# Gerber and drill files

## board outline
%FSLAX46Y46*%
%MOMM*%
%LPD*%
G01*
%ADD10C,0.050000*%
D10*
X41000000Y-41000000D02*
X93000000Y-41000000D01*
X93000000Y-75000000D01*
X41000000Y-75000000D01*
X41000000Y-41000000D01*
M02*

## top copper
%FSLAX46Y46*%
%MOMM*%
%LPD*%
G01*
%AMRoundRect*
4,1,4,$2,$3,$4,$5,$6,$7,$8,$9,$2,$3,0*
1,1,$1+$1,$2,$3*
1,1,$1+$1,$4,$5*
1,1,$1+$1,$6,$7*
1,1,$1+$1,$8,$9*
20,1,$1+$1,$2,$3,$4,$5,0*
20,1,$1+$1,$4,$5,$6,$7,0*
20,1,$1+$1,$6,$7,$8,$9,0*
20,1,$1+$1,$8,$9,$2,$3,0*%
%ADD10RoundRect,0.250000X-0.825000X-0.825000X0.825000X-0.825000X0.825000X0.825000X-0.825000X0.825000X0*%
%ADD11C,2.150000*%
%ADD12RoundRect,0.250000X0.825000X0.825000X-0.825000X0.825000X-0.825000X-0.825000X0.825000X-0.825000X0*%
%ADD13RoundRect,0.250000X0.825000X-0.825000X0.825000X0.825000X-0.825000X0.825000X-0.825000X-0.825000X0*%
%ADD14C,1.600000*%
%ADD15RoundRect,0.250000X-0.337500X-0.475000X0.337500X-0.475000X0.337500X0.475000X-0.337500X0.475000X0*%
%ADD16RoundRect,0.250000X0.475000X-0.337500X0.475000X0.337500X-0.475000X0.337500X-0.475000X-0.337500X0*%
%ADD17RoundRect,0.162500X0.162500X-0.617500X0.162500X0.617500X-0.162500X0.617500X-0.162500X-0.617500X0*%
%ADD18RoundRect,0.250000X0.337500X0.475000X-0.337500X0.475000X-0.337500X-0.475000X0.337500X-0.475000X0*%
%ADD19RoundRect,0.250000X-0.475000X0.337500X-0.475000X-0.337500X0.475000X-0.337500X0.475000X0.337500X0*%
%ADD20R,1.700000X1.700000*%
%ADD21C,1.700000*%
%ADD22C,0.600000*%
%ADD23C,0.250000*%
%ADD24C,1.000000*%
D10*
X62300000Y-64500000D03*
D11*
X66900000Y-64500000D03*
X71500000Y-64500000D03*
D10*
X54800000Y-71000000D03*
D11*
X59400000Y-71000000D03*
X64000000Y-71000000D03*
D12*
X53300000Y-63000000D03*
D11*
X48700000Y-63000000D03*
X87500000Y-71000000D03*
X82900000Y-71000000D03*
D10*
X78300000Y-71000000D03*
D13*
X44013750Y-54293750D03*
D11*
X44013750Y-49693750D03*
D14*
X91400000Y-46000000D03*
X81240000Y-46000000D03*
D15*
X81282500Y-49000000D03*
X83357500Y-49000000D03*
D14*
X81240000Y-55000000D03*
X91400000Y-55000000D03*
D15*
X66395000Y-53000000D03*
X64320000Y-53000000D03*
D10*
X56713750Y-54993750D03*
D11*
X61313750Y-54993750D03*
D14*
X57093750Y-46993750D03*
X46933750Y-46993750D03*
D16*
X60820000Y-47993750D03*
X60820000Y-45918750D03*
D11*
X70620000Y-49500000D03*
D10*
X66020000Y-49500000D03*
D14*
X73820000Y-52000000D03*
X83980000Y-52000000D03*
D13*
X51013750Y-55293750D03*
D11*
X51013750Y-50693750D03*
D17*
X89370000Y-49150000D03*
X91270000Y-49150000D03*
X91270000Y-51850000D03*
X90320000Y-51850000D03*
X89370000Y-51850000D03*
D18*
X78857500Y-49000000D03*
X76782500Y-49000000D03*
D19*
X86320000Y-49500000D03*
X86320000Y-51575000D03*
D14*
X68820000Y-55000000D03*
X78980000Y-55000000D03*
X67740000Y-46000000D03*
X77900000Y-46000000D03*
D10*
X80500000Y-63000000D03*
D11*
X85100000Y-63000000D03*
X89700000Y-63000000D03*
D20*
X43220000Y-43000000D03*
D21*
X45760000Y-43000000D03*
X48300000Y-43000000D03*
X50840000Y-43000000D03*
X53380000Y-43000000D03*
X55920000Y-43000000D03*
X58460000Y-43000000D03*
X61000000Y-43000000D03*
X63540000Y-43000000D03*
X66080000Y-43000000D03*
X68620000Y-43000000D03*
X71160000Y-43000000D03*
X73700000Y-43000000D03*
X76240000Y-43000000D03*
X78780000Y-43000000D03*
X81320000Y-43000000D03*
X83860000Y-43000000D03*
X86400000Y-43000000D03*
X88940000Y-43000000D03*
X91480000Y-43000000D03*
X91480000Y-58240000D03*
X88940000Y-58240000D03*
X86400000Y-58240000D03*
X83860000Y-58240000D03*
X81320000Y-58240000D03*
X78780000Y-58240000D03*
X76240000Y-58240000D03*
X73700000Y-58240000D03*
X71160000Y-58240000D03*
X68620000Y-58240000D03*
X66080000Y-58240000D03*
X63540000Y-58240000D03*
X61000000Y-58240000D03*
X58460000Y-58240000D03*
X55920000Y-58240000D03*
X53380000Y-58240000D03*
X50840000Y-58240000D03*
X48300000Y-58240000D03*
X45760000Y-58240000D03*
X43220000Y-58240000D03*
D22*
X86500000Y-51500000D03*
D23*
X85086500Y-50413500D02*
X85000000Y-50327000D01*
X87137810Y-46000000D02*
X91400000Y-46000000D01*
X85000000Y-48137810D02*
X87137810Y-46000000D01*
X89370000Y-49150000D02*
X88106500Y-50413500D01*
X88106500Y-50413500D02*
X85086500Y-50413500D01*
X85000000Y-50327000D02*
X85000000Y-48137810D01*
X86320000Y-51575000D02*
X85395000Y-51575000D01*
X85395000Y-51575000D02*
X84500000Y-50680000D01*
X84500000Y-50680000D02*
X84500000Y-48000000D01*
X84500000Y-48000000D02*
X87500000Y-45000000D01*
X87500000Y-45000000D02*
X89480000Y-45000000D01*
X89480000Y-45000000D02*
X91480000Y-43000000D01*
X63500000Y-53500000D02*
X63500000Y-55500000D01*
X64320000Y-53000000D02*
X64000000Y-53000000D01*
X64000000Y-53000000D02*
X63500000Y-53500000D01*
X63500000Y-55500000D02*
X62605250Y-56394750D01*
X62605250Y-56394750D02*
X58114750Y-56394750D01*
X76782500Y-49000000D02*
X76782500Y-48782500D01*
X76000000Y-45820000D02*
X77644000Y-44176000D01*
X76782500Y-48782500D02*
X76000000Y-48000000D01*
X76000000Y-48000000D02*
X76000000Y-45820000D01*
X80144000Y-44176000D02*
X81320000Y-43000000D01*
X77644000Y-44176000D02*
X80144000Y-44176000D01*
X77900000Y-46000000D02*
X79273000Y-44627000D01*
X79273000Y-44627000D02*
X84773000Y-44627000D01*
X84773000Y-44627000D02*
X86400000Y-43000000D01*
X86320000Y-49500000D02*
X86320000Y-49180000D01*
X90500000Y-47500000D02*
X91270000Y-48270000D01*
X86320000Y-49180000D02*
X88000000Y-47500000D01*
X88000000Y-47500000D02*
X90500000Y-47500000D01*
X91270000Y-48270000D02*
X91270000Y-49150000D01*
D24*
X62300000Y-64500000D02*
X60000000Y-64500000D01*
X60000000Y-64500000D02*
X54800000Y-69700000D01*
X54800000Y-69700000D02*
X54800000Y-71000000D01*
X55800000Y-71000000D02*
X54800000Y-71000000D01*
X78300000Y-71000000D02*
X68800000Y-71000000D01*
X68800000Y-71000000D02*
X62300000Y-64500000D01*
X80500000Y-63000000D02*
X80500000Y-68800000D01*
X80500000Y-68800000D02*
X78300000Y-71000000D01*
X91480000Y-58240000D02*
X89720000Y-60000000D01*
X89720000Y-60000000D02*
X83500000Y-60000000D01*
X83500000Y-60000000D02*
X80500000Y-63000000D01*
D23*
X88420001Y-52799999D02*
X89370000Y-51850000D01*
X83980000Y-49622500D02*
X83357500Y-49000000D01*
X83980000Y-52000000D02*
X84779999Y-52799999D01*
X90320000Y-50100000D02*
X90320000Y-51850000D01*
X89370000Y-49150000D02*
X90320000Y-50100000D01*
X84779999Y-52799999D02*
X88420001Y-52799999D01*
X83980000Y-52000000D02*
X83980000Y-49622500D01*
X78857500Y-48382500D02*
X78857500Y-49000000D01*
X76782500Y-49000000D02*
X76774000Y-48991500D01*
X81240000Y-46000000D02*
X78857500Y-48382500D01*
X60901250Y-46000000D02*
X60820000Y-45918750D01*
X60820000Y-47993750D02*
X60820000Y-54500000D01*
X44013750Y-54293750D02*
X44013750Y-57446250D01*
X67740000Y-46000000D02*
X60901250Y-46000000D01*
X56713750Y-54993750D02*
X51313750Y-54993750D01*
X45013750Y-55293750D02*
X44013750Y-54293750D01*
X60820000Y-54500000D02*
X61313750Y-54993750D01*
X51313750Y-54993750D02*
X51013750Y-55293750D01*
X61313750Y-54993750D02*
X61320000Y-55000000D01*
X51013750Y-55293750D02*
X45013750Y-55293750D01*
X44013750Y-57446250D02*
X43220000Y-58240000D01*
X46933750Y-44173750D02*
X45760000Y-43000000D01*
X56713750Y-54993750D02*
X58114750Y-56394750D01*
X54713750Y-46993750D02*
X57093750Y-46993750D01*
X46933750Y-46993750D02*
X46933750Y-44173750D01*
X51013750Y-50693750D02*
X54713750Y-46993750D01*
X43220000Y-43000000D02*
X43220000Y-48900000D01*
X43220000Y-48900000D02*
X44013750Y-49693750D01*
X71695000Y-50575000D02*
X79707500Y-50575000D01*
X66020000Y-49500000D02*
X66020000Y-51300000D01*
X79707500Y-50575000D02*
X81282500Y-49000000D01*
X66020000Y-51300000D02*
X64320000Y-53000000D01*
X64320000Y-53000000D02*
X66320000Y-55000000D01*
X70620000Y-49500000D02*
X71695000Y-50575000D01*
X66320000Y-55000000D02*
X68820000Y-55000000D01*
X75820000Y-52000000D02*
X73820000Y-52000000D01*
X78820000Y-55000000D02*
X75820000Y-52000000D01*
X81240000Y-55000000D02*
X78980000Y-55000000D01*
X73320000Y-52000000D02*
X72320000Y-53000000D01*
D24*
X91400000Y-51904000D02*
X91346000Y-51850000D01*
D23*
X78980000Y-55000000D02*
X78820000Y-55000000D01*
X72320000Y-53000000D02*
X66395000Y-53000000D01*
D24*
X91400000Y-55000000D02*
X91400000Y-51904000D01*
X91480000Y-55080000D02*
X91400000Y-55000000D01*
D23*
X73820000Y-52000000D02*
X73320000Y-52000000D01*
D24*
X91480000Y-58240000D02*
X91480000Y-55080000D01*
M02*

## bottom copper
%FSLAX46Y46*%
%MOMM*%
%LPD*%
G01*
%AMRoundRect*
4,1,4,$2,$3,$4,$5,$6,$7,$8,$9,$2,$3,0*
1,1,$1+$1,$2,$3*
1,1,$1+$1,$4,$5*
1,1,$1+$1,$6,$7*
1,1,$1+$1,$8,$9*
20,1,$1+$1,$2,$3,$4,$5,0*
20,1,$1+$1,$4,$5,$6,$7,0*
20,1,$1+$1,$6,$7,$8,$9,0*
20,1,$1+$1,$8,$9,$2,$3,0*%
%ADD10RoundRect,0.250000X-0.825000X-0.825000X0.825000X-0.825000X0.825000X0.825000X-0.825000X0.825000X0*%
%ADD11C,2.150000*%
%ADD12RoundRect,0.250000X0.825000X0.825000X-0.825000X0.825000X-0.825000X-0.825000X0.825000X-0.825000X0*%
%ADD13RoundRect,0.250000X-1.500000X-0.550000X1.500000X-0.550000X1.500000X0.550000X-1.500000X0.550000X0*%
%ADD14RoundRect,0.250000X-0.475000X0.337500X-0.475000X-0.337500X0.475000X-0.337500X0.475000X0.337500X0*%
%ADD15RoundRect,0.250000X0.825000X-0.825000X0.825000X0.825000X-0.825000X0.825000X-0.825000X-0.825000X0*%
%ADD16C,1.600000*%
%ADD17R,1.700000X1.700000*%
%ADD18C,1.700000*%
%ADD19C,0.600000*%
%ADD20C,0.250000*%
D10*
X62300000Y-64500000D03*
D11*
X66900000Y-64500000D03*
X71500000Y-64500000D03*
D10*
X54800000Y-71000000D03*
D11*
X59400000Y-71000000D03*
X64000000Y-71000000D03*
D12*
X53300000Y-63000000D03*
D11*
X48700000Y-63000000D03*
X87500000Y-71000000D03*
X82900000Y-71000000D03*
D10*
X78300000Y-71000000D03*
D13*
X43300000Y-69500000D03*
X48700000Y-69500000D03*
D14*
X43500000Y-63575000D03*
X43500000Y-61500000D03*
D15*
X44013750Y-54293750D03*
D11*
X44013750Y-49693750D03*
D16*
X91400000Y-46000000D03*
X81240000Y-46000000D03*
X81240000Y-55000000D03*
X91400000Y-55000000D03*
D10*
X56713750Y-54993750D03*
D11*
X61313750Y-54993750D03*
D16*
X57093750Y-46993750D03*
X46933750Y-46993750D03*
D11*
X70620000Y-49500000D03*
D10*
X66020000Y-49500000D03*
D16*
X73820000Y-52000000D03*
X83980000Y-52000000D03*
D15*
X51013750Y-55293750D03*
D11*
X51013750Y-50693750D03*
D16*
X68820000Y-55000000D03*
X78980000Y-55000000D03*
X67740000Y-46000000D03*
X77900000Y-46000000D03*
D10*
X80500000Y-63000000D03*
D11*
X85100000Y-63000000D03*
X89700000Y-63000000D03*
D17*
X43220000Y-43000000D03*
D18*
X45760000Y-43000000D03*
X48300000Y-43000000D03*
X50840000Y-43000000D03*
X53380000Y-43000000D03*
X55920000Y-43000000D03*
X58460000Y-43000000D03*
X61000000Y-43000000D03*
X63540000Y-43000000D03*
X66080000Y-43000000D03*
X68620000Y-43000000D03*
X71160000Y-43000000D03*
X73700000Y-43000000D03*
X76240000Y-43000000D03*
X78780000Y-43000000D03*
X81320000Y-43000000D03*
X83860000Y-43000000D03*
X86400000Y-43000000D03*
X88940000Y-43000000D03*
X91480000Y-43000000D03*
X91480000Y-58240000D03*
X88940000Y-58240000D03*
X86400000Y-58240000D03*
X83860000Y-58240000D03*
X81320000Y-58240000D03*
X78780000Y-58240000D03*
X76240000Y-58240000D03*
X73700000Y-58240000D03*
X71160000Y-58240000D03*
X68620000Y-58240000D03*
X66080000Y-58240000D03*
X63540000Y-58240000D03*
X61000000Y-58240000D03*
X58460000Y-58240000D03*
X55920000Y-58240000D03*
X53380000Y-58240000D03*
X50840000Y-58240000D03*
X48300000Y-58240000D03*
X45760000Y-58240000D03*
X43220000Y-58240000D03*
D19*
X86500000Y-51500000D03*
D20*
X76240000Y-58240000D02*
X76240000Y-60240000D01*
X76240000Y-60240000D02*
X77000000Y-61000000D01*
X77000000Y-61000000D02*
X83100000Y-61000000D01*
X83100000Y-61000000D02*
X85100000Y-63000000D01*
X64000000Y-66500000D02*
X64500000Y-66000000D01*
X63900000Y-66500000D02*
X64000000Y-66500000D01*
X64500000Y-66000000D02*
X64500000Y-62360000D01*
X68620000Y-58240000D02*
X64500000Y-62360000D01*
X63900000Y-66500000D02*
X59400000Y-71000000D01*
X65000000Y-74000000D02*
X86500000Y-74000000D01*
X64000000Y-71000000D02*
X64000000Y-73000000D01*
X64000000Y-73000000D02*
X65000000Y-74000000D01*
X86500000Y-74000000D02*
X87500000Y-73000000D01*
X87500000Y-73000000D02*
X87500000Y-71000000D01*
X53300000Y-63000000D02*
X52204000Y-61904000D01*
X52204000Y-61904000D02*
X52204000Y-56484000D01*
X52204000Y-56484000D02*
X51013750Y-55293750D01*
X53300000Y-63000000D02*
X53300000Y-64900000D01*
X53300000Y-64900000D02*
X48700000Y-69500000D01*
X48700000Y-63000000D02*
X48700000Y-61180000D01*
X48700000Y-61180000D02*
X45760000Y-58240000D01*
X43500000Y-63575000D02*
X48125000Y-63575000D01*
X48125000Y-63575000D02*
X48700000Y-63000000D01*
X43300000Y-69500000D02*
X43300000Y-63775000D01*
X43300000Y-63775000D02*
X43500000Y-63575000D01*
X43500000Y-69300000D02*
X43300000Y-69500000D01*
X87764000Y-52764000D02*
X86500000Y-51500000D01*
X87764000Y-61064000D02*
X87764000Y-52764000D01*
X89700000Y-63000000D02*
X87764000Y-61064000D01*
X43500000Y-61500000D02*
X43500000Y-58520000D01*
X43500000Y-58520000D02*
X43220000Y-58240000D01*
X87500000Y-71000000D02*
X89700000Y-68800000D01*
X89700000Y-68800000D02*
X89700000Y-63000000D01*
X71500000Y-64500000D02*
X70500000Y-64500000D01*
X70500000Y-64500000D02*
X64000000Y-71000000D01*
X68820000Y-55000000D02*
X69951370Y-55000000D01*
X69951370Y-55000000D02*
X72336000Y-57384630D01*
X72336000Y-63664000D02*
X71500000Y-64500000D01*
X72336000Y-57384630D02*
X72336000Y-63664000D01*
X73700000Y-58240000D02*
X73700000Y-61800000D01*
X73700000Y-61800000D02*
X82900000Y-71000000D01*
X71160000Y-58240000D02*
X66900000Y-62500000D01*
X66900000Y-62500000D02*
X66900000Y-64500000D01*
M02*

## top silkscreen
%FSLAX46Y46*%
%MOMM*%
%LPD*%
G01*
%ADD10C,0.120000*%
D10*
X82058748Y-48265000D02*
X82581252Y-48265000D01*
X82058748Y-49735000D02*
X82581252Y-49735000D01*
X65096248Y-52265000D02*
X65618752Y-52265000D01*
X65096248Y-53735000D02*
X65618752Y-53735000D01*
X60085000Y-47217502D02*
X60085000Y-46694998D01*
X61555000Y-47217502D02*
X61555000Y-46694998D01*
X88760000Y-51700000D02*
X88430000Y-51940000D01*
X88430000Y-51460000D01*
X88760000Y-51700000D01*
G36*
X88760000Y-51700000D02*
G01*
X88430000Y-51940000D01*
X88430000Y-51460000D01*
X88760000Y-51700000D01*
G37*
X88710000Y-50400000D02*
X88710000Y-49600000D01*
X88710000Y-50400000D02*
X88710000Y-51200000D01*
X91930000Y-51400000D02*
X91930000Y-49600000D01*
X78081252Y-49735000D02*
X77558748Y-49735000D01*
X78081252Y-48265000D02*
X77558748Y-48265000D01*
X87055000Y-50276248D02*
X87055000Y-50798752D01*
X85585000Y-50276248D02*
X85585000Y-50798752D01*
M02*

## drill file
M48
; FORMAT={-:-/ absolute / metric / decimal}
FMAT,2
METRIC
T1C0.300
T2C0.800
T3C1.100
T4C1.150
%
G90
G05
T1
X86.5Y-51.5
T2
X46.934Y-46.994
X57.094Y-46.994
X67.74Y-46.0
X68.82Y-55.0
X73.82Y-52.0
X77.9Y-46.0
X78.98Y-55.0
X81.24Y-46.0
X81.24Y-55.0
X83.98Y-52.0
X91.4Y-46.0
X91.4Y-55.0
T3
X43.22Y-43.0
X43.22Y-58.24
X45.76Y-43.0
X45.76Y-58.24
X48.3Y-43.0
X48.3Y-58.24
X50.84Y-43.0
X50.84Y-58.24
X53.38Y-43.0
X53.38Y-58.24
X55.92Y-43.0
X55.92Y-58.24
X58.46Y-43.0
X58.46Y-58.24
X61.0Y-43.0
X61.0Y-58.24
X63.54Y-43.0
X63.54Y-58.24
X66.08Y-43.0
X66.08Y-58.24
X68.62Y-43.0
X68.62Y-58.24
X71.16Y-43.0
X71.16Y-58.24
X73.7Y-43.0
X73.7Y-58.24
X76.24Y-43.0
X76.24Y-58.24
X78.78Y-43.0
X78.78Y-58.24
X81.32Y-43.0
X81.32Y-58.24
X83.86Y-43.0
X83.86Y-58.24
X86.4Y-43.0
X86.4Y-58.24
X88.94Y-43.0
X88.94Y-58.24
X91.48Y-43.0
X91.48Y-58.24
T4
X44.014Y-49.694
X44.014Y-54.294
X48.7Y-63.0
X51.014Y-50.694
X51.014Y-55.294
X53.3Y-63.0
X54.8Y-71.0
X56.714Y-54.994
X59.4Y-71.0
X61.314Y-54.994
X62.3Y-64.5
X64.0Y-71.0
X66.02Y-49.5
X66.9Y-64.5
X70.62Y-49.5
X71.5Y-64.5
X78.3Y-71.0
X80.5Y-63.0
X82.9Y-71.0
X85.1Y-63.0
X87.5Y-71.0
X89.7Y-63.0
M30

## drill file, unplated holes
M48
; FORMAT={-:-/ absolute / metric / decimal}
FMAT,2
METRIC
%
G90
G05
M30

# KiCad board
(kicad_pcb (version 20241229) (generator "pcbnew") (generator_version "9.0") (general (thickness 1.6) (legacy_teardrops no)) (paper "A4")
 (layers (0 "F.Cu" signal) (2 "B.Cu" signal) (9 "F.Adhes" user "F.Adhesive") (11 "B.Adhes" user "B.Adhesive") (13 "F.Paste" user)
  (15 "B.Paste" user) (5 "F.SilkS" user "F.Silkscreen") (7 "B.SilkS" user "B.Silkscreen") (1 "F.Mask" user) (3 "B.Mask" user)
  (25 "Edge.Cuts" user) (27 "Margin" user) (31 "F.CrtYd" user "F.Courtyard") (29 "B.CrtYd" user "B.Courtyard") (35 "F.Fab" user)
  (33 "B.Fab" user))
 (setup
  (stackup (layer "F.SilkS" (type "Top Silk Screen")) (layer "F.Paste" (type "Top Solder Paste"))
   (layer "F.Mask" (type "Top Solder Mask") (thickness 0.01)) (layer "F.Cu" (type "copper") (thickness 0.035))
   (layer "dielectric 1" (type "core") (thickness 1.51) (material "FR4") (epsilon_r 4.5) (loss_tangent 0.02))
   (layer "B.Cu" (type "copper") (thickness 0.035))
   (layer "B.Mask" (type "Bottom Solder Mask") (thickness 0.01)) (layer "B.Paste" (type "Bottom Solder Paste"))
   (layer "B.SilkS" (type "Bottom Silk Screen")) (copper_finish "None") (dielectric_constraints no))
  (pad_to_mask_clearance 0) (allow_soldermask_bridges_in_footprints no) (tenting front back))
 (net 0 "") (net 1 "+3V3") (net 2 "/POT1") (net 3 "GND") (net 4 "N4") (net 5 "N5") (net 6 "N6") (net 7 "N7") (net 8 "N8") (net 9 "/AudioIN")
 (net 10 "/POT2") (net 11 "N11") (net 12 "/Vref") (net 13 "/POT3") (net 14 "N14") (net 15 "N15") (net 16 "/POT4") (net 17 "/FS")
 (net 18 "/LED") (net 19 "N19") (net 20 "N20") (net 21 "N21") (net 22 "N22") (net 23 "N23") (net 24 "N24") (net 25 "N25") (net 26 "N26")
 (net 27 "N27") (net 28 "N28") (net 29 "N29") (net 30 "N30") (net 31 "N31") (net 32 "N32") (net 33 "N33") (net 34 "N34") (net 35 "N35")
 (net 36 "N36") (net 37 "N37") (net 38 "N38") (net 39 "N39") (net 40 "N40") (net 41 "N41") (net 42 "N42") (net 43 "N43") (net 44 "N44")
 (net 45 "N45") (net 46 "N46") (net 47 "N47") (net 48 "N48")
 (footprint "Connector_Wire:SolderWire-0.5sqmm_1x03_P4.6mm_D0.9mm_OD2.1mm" (layer "F.Cu") (at 54.8 71)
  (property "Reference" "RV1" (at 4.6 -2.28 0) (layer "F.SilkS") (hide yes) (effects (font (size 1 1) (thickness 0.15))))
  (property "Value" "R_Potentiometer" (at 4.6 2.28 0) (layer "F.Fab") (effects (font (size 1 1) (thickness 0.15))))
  (pad "1" thru_hole roundrect (at 0 0) (size 2.15 2.15) (drill 1.15) (layers "*.Cu" "*.Mask") (remove_unused_layers no)
   (roundrect_rratio 0.116279) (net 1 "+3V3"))
  (pad "2" thru_hole circle (at 4.6 0) (size 2.15 2.15) (drill 1.15) (layers "*.Cu" "*.Mask") (remove_unused_layers no) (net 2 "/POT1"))
  (pad "3" thru_hole circle (at 9.2 0) (size 2.15 2.15) (drill 1.15) (layers "*.Cu" "*.Mask") (remove_unused_layers no) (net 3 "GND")))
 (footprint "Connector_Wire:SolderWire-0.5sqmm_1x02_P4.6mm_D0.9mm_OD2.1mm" (layer "F.Cu") (at 53.3 63 180)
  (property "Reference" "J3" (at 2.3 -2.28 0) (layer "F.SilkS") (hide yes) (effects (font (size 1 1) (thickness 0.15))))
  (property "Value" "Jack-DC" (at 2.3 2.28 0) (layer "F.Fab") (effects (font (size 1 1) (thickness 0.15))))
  (pad "1" thru_hole roundrect (at 0 0 180) (size 2.15 2.15) (drill 1.15) (layers "*.Cu" "*.Mask") (remove_unused_layers no)
   (roundrect_rratio 0.116279) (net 3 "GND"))
  (pad "2" thru_hole circle (at 4.6 0 180) (size 2.15 2.15) (drill 1.15) (layers "*.Cu" "*.Mask") (remove_unused_layers no) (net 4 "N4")))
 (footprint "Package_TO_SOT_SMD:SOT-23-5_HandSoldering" (layer "F.Cu") (at 90.32 50.5 90)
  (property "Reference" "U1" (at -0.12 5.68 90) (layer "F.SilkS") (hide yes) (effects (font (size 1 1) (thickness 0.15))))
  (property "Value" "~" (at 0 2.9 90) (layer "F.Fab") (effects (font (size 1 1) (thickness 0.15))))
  (fp_line (start 0.1 -1.61) (end 0.9 -1.61) (stroke (width 0.12) (type solid)) (layer "F.SilkS"))
  (fp_line (start 0.1 -1.61) (end -0.7 -1.61) (stroke (width 0.12) (type solid)) (layer "F.SilkS"))
  (fp_line (start -0.9 1.61) (end 0.9 1.61) (stroke (width 0.12) (type solid)) (layer "F.SilkS"))
  (fp_poly
   (pts (xy -1.2 -1.56) (xy -1.44 -1.89) (xy -0.96 -1.89) (xy -1.2 -1.56)) (stroke (width 0.12) (type solid)) (fill yes) (layer "F.SilkS"))
  (pad "1" smd roundrect (at -1.35 -0.95 90) (size 1.56 0.65) (layers "F.Cu" "F.Mask" "F.Paste") (roundrect_rratio 0.25) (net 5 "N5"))
  (pad "2" smd roundrect (at -1.35 0 90) (size 1.56 0.65) (layers "F.Cu" "F.Mask" "F.Paste") (roundrect_rratio 0.25) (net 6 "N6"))
  (pad "3" smd roundrect (at -1.35 0.95 90) (size 1.56 0.65) (layers "F.Cu" "F.Mask" "F.Paste") (roundrect_rratio 0.25) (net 1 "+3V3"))
  (pad "4" smd roundrect (at 1.35 0.95 90) (size 1.56 0.65) (layers "F.Cu" "F.Mask" "F.Paste") (roundrect_rratio 0.25) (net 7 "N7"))
  (pad "5" smd roundrect (at 1.35 -0.95 90) (size 1.56 0.65) (layers "F.Cu" "F.Mask" "F.Paste") (roundrect_rratio 0.25) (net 6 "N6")))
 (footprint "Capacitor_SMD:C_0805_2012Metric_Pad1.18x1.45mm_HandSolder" (layer "F.Cu") (at 77.82 49 180)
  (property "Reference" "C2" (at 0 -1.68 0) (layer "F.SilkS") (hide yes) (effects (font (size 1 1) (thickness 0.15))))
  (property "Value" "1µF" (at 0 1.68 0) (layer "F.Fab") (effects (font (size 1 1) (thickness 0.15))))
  (fp_line (start -0.261252 0.735) (end 0.261252 0.735) (stroke (width 0.12) (type solid)) (layer "F.SilkS"))
  (fp_line (start -0.261252 -0.735) (end 0.261252 -0.735) (stroke (width 0.12) (type solid)) (layer "F.SilkS"))
  (pad "1" smd roundrect (at -1.0375 0 180) (size 1.175 1.45) (layers "F.Cu" "F.Mask" "F.Paste") (roundrect_rratio 0.212766) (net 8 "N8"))
  (pad "2" smd roundrect (at 1.0375 0 180) (size 1.175 1.45) (layers "F.Cu" "F.Mask" "F.Paste") (roundrect_rratio 0.212766)
   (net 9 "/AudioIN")))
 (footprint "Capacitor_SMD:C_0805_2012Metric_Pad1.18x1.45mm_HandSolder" (layer "F.Cu") (at 86.32 50.5375 -90)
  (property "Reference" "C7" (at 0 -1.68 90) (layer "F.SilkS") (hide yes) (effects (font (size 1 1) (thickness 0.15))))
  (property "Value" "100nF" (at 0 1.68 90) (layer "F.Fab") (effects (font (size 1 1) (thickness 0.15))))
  (fp_line (start -0.261252 0.735) (end 0.261252 0.735) (stroke (width 0.12) (type solid)) (layer "F.SilkS"))
  (fp_line (start -0.261252 -0.735) (end 0.261252 -0.735) (stroke (width 0.12) (type solid)) (layer "F.SilkS"))
  (pad "1" smd roundrect (at -1.0375 0 270) (size 1.175 1.45) (layers "F.Cu" "F.Mask" "F.Paste") (roundrect_rratio 0.212766) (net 7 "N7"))
  (pad "2" smd roundrect (at 1.0375 0 270) (size 1.175 1.45) (layers "F.Cu" "F.Mask" "F.Paste") (roundrect_rratio 0.212766) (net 3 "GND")))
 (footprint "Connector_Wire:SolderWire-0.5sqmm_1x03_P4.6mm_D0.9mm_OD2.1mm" (layer "F.Cu") (at 62.3 64.5)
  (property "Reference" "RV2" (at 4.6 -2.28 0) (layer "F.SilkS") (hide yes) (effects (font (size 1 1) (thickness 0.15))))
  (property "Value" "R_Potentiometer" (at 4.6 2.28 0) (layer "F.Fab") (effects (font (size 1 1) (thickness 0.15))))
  (pad "1" thru_hole roundrect (at 0 0) (size 2.15 2.15) (drill 1.15) (layers "*.Cu" "*.Mask") (remove_unused_layers no)
   (roundrect_rratio 0.116279) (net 1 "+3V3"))
  (pad "2" thru_hole circle (at 4.6 0) (size 2.15 2.15) (drill 1.15) (layers "*.Cu" "*.Mask") (remove_unused_layers no) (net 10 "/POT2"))
  (pad "3" thru_hole circle (at 9.2 0) (size 2.15 2.15) (drill 1.15) (layers "*.Cu" "*.Mask") (remove_unused_layers no) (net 3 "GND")))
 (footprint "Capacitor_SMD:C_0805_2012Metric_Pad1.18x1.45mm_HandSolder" (layer "F.Cu") (at 82.32 49)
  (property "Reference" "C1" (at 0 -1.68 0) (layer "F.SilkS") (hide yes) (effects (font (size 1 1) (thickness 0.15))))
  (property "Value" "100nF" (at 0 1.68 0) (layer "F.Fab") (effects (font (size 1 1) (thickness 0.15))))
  (fp_line (start -0.261252 -0.735) (end 0.261252 -0.735) (stroke (width 0.12) (type solid)) (layer "F.SilkS"))
  (fp_line (start -0.261252 0.735) (end 0.261252 0.735) (stroke (width 0.12) (type solid)) (layer "F.SilkS"))
  (pad "1" smd roundrect (at -1.0375 0) (size 1.175 1.45) (layers "F.Cu" "F.Mask" "F.Paste") (roundrect_rratio 0.212766) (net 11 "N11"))
  (pad "2" smd roundrect (at 1.0375 0) (size 1.175 1.45) (layers "F.Cu" "F.Mask" "F.Paste") (roundrect_rratio 0.212766) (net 5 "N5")))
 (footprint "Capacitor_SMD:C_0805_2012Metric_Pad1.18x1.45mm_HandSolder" (layer "F.Cu") (at 65.3575 53)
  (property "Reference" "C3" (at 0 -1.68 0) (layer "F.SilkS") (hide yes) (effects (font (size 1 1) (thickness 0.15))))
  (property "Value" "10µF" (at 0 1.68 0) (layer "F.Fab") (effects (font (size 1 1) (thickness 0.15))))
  (fp_line (start -0.261252 -0.735) (end 0.261252 -0.735) (stroke (width 0.12) (type solid)) (layer "F.SilkS"))
  (fp_line (start -0.261252 0.735) (end 0.261252 0.735) (stroke (width 0.12) (type solid)) (layer "F.SilkS"))
  (pad "1" smd roundrect (at -1.0375 0) (size 1.175 1.45) (layers "F.Cu" "F.Mask" "F.Paste") (roundrect_rratio 0.212766) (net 3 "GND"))
  (pad "2" smd roundrect (at 1.0375 0) (size 1.175 1.45) (layers "F.Cu" "F.Mask" "F.Paste") (roundrect_rratio 0.212766) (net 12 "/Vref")))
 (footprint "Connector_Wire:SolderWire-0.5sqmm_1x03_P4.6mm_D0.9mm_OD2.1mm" (layer "F.Cu") (at 78.3 71)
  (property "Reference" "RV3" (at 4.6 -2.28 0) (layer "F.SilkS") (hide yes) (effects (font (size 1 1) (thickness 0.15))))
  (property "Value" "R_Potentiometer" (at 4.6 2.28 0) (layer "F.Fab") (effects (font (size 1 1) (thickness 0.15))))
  (pad "1" thru_hole roundrect (at 0 0) (size 2.15 2.15) (drill 1.15) (layers "*.Cu" "*.Mask") (remove_unused_layers no)
   (roundrect_rratio 0.116279) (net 1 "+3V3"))
  (pad "2" thru_hole circle (at 4.6 0) (size 2.15 2.15) (drill 1.15) (layers "*.Cu" "*.Mask") (remove_unused_layers no) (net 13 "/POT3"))
  (pad "3" thru_hole circle (at 9.2 0) (size 2.15 2.15) (drill 1.15) (layers "*.Cu" "*.Mask") (remove_unused_layers no) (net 3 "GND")))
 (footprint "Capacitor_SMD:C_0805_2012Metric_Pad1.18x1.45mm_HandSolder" (layer "F.Cu") (at 60.82 46.95625 90)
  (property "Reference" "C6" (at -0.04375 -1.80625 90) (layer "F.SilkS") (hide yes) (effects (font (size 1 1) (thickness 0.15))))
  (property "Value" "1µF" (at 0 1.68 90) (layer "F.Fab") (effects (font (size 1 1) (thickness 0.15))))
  (fp_line (start -0.261252 -0.735) (end 0.261252 -0.735) (stroke (width 0.12) (type solid)) (layer "F.SilkS"))
  (fp_line (start -0.261252 0.735) (end 0.261252 0.735) (stroke (width 0.12) (type solid)) (layer "F.SilkS"))
  (pad "1" smd roundrect (at -1.0375 0 90) (size 1.175 1.45) (layers "F.Cu" "F.Mask" "F.Paste") (roundrect_rratio 0.212766) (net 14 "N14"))
  (pad "2" smd roundrect (at 1.0375 0 90) (size 1.175 1.45) (layers "F.Cu" "F.Mask" "F.Paste") (roundrect_rratio 0.212766) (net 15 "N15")))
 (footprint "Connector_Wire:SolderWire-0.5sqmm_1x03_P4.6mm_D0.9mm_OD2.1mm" (layer "F.Cu") (at 80.5 63)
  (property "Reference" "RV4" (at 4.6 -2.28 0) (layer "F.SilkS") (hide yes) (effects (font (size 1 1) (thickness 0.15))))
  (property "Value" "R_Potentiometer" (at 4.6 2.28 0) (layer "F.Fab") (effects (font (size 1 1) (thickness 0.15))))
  (pad "1" thru_hole roundrect (at 0 0) (size 2.15 2.15) (drill 1.15) (layers "*.Cu" "*.Mask") (remove_unused_layers no)
   (roundrect_rratio 0.116279) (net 1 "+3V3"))
  (pad "2" thru_hole circle (at 4.6 0) (size 2.15 2.15) (drill 1.15) (layers "*.Cu" "*.Mask") (remove_unused_layers no) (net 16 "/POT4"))
  (pad "3" thru_hole circle (at 9.2 0) (size 2.15 2.15) (drill 1.15) (layers "*.Cu" "*.Mask") (remove_unused_layers no) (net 3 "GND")))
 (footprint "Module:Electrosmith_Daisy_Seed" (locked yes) (layer "B.Cu") (at 43.22 43 -90)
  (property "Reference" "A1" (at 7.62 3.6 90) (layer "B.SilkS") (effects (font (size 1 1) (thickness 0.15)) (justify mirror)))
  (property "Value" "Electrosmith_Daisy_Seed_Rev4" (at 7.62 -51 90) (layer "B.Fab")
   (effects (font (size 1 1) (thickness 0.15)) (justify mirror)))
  (pad "1" thru_hole rect (at 0 0 270) (size 1.7 1.7) (drill 1.1) (layers "*.Cu" "*.Mask") (remove_unused_layers no) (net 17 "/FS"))
  (pad "2" thru_hole circle (at 0 -2.54 270) (size 1.7 1.7) (drill 1.1) (layers "*.Cu" "*.Mask") (remove_unused_layers no) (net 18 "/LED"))
  (pad "3" thru_hole circle (at 0 -5.08 270) (size 1.7 1.7) (drill 1.1) (layers "*.Cu" "*.Mask") (remove_unused_layers no) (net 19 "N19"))
  (pad "4" thru_hole circle (at 0 -7.62 270) (size 1.7 1.7) (drill 1.1) (layers "*.Cu" "*.Mask") (remove_unused_layers no) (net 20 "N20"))
  (pad "5" thru_hole circle (at 0 -10.16 270) (size 1.7 1.7) (drill 1.1) (layers "*.Cu" "*.Mask") (remove_unused_layers no) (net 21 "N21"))
  (pad "6" thru_hole circle (at 0 -12.7 270) (size 1.7 1.7) (drill 1.1) (layers "*.Cu" "*.Mask") (remove_unused_layers no) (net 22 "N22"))
  (pad "7" thru_hole circle (at 0 -15.24 270) (size 1.7 1.7) (drill 1.1) (layers "*.Cu" "*.Mask") (remove_unused_layers no) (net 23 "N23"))
  (pad "8" thru_hole circle (at 0 -17.78 270) (size 1.7 1.7) (drill 1.1) (layers "*.Cu" "*.Mask") (remove_unused_layers no) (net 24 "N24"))
  (pad "9" thru_hole circle (at 0 -20.32 270) (size 1.7 1.7) (drill 1.1) (layers "*.Cu" "*.Mask") (remove_unused_layers no) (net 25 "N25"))
  (pad "10" thru_hole circle (at 0 -22.86 270) (size 1.7 1.7) (drill 1.1) (layers "*.Cu" "*.Mask") (remove_unused_layers no) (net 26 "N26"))
  (pad "11" thru_hole circle (at 0 -25.4 270) (size 1.7 1.7) (drill 1.1) (layers "*.Cu" "*.Mask") (remove_unused_layers no) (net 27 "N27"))
  (pad "12" thru_hole circle (at 0 -27.94 270) (size 1.7 1.7) (drill 1.1) (layers "*.Cu" "*.Mask") (remove_unused_layers no) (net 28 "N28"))
  (pad "13" thru_hole circle (at 0 -30.48 270) (size 1.7 1.7) (drill 1.1) (layers "*.Cu" "*.Mask") (remove_unused_layers no) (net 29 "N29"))
  (pad "14" thru_hole circle (at 0 -33.02 270) (size 1.7 1.7) (drill 1.1) (layers "*.Cu" "*.Mask") (remove_unused_layers no) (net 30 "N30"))
  (pad "15" thru_hole circle (at 0 -35.56 270) (size 1.7 1.7) (drill 1.1) (layers "*.Cu" "*.Mask") (remove_unused_layers no) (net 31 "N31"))
  (pad "16" thru_hole circle (at 0 -38.1 270) (size 1.7 1.7) (drill 1.1) (layers "*.Cu" "*.Mask") (remove_unused_layers no)
   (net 9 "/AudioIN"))
  (pad "17" thru_hole circle (at 0 -40.64 270) (size 1.7 1.7) (drill 1.1) (layers "*.Cu" "*.Mask") (remove_unused_layers no) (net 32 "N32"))
  (pad "18" thru_hole circle (at 0 -43.18 270) (size 1.7 1.7) (drill 1.1) (layers "*.Cu" "*.Mask") (remove_unused_layers no) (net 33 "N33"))
  (pad "19" thru_hole circle (at 0 -45.72 270) (size 1.7 1.7) (drill 1.1) (layers "*.Cu" "*.Mask") (remove_unused_layers no) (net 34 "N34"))
  (pad "20" thru_hole circle (at 0 -48.26 270) (size 1.7 1.7) (drill 1.1) (layers "*.Cu" "*.Mask") (remove_unused_layers no) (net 3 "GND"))
  (pad "21" thru_hole circle (at 15.24 -48.26 270) (size 1.7 1.7) (drill 1.1) (layers "*.Cu" "*.Mask") (remove_unused_layers no)
   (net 1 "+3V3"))
  (pad "22" thru_hole circle (at 15.24 -45.72 270) (size 1.7 1.7) (drill 1.1) (layers "*.Cu" "*.Mask") (remove_unused_layers no)
   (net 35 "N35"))
  (pad "23" thru_hole circle (at 15.24 -43.18 270) (size 1.7 1.7) (drill 1.1) (layers "*.Cu" "*.Mask") (remove_unused_layers no)
   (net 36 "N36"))
  (pad "24" thru_hole circle (at 15.24 -40.64 270) (size 1.7 1.7) (drill 1.1) (layers "*.Cu" "*.Mask") (remove_unused_layers no)
   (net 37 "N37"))
  (pad "25" thru_hole circle (at 15.24 -38.1 270) (size 1.7 1.7) (drill 1.1) (layers "*.Cu" "*.Mask") (remove_unused_layers no)
   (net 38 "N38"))
  (pad "26" thru_hole circle (at 15.24 -35.56 270) (size 1.7 1.7) (drill 1.1) (layers "*.Cu" "*.Mask") (remove_unused_layers no)
   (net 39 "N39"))
  (pad "27" thru_hole circle (at 15.24 -33.02 270) (size 1.7 1.7) (drill 1.1) (layers "*.Cu" "*.Mask") (remove_unused_layers no)
   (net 16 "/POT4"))
  (pad "28" thru_hole circle (at 15.24 -30.48 270) (size 1.7 1.7) (drill 1.1) (layers "*.Cu" "*.Mask") (remove_unused_layers no)
   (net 13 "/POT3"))
  (pad "29" thru_hole circle (at 15.24 -27.94 270) (size 1.7 1.7) (drill 1.1) (layers "*.Cu" "*.Mask") (remove_unused_layers no)
   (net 10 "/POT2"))
  (pad "30" thru_hole circle (at 15.24 -25.4 270) (size 1.7 1.7) (drill 1.1) (layers "*.Cu" "*.Mask") (remove_unused_layers no)
   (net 2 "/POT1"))
  (pad "31" thru_hole circle (at 15.24 -22.86 270) (size 1.7 1.7) (drill 1.1) (layers "*.Cu" "*.Mask") (remove_unused_layers no)
   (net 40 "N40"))
  (pad "32" thru_hole circle (at 15.24 -20.32 270) (size 1.7 1.7) (drill 1.1) (layers "*.Cu" "*.Mask") (remove_unused_layers no)
   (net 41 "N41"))
  (pad "33" thru_hole circle (at 15.24 -17.78 270) (size 1.7 1.7) (drill 1.1) (layers "*.Cu" "*.Mask") (remove_unused_layers no)
   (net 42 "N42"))
  (pad "34" thru_hole circle (at 15.24 -15.24 270) (size 1.7 1.7) (drill 1.1) (layers "*.Cu" "*.Mask") (remove_unused_layers no)
   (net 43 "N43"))
  (pad "35" thru_hole circle (at 15.24 -12.7 270) (size 1.7 1.7) (drill 1.1) (layers "*.Cu" "*.Mask") (remove_unused_layers no)
   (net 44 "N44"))
  (pad "36" thru_hole circle (at 15.24 -10.16 270) (size 1.7 1.7) (drill 1.1) (layers "*.Cu" "*.Mask") (remove_unused_layers no)
   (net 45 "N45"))
  (pad "37" thru_hole circle (at 15.24 -7.62 270) (size 1.7 1.7) (drill 1.1) (layers "*.Cu" "*.Mask") (remove_unused_layers no)
   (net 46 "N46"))
  (pad "38" thru_hole circle (at 15.24 -5.08 270) (size 1.7 1.7) (drill 1.1) (layers "*.Cu" "*.Mask") (remove_unused_layers no)
   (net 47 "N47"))
  (pad "39" thru_hole circle (at 15.24 -2.54 270) (size 1.7 1.7) (drill 1.1) (layers "*.Cu" "*.Mask") (remove_unused_layers no) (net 4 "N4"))
  (pad "40" thru_hole circle (at 15.24 0 270) (size 1.7 1.7) (drill 1.1) (layers "*.Cu" "*.Mask") (remove_unused_layers no) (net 3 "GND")))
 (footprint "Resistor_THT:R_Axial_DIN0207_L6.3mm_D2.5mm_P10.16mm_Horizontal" (layer "B.Cu") (at 73.82 52)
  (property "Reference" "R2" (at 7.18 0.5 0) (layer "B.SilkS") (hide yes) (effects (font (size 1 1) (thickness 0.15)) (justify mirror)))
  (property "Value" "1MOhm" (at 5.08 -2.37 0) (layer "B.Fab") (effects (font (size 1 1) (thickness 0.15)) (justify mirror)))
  (pad "1" thru_hole circle (at 0 0) (size 1.6 1.6) (drill 0.8) (layers "*.Cu" "*.Mask") (remove_unused_layers no) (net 12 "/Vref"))
  (pad "2" thru_hole circle (at 10.16 0) (size 1.6 1.6) (drill 0.8) (layers "*.Cu" "*.Mask") (remove_unused_layers no) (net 5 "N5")))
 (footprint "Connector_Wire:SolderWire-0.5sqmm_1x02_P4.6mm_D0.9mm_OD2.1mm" (layer "B.Cu") (at 51.01375 55.29375 90)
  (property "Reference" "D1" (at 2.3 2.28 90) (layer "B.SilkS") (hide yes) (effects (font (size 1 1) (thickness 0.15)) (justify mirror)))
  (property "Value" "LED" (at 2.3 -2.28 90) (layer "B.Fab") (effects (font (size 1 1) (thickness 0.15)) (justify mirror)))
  (pad "1" thru_hole roundrect (at 0 0 90) (size 2.15 2.15) (drill 1.15) (layers "*.Cu" "*.Mask") (remove_unused_layers no)
   (roundrect_rratio 0.116279) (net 3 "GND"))
  (pad "2" thru_hole circle (at 4.6 0 90) (size 2.15 2.15) (drill 1.15) (layers "*.Cu" "*.Mask") (remove_unused_layers no) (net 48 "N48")))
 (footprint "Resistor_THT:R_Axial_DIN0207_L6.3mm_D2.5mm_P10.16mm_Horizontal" (layer "B.Cu") (at 68.82 55)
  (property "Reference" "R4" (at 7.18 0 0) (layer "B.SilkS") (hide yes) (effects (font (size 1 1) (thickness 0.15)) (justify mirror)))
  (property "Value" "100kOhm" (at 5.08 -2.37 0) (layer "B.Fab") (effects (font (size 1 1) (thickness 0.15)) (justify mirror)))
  (pad "1" thru_hole circle (at 0 0) (size 1.6 1.6) (drill 0.8) (layers "*.Cu" "*.Mask") (remove_unused_layers no) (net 3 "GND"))
  (pad "2" thru_hole circle (at 10.16 0) (size 1.6 1.6) (drill 0.8) (layers "*.Cu" "*.Mask") (remove_unused_layers no) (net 12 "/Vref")))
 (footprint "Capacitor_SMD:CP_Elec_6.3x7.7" (layer "B.Cu") (at 46 69.5)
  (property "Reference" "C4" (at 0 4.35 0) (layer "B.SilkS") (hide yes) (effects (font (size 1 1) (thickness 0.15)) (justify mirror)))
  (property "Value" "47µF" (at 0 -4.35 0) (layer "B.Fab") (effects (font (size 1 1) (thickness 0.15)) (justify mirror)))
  (pad "1" smd roundrect (at -2.7 0) (size 3.5 1.6) (layers "B.Cu" "B.Mask" "B.Paste") (roundrect_rratio 0.15625) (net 4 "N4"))
  (pad "2" smd roundrect (at 2.7 0) (size 3.5 1.6) (layers "B.Cu" "B.Mask" "B.Paste") (roundrect_rratio 0.15625) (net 3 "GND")))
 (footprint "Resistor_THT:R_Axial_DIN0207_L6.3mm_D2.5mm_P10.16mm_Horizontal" (layer "B.Cu") (at 67.74 46)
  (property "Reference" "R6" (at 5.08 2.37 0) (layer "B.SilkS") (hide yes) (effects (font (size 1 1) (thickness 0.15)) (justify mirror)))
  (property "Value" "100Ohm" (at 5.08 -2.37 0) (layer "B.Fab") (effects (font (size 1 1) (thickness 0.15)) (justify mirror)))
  (pad "1" thru_hole circle (at 0 0) (size 1.6 1.6) (drill 0.8) (layers "*.Cu" "*.Mask") (remove_unused_layers no) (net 15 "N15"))
  (pad "2" thru_hole circle (at 10.16 0) (size 1.6 1.6) (drill 0.8) (layers "*.Cu" "*.Mask") (remove_unused_layers no) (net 33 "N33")))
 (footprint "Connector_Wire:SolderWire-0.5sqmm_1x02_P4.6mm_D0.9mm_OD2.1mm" (layer "B.Cu") (at 44.01375 54.29375 90)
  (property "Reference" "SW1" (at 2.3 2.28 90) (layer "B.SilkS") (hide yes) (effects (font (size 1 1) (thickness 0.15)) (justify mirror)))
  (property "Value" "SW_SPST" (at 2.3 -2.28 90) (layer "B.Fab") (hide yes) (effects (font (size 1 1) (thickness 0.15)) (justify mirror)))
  (pad "1" thru_hole roundrect (at 0 0 90) (size 2.15 2.15) (drill 1.15) (layers "*.Cu" "*.Mask") (remove_unused_layers no)
   (roundrect_rratio 0.116279) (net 3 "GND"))
  (pad "2" thru_hole circle (at 4.6 0 90) (size 2.15 2.15) (drill 1.15) (layers "*.Cu" "*.Mask") (remove_unused_layers no) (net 17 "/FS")))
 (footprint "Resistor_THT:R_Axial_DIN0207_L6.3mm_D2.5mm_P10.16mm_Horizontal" (layer "B.Cu") (at 91.4 46 180)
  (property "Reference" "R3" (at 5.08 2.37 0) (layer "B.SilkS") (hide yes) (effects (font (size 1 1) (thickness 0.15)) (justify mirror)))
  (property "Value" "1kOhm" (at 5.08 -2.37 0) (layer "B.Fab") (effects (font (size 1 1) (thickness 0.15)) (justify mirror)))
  (pad "1" thru_hole circle (at 0 0 180) (size 1.6 1.6) (drill 0.8) (layers "*.Cu" "*.Mask") (remove_unused_layers no) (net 6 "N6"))
  (pad "2" thru_hole circle (at 10.16 0 180) (size 1.6 1.6) (drill 0.8) (layers "*.Cu" "*.Mask") (remove_unused_layers no) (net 8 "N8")))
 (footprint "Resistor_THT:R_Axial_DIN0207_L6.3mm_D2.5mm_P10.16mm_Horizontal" (layer "B.Cu") (at 81.24 55)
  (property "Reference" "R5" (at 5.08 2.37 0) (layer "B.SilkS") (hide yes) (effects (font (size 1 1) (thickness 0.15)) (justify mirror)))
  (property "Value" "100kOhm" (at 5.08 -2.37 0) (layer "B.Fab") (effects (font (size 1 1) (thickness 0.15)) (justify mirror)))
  (pad "1" thru_hole circle (at 0 0) (size 1.6 1.6) (drill 0.8) (layers "*.Cu" "*.Mask") (remove_unused_layers no) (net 12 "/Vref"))
  (pad "2" thru_hole circle (at 10.16 0) (size 1.6 1.6) (drill 0.8) (layers "*.Cu" "*.Mask") (remove_unused_layers no) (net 1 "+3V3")))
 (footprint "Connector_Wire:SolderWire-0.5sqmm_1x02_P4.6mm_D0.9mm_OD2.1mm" (layer "B.Cu") (at 56.71375 54.99375)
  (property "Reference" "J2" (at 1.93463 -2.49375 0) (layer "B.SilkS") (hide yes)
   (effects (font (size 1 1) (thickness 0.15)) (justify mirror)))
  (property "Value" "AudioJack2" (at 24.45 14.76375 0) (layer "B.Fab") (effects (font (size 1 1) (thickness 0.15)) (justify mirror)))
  (pad "S" thru_hole roundrect (at 0 0) (size 2.15 2.15) (drill 1.15) (layers "*.Cu" "*.Mask") (remove_unused_layers no)
   (roundrect_rratio 0.116279) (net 3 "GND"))
  (pad "T" thru_hole circle (at 4.6 0) (size 2.15 2.15) (drill 1.15) (layers "*.Cu" "*.Mask") (remove_unused_layers no) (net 14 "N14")))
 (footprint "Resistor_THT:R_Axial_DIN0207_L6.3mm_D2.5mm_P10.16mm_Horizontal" (layer "B.Cu") (at 57.09375 46.99375 180)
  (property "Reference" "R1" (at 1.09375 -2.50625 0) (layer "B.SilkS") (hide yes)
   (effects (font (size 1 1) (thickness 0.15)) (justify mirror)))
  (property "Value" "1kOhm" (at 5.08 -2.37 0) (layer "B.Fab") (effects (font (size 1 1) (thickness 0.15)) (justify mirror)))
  (pad "1" thru_hole circle (at 0 0 180) (size 1.6 1.6) (drill 0.8) (layers "*.Cu" "*.Mask") (remove_unused_layers no) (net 48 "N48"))
  (pad "2" thru_hole circle (at 10.16 0 180) (size 1.6 1.6) (drill 0.8) (layers "*.Cu" "*.Mask") (remove_unused_layers no) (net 18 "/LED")))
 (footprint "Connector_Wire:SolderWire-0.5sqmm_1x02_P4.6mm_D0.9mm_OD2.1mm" (layer "B.Cu") (at 66.02 49.5)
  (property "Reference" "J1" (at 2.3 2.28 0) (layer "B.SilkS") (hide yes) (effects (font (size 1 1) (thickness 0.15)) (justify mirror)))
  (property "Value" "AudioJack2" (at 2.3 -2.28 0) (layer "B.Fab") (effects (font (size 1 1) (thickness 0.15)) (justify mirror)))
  (pad "S" thru_hole roundrect (at 0 0) (size 2.15 2.15) (drill 1.15) (layers "*.Cu" "*.Mask") (remove_unused_layers no)
   (roundrect_rratio 0.116279) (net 3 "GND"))
  (pad "T" thru_hole circle (at 4.6 0) (size 2.15 2.15) (drill 1.15) (layers "*.Cu" "*.Mask") (remove_unused_layers no) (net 11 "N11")))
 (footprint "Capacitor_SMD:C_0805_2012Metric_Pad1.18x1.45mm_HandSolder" (layer "B.Cu") (at 43.5 62.5375 -90)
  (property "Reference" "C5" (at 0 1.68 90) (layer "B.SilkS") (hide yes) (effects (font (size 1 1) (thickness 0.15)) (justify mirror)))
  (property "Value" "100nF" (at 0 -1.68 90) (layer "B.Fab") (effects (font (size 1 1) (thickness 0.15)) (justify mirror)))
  (pad "1" smd roundrect (at -1.0375 0 270) (size 1.175 1.45) (layers "B.Cu" "B.Mask" "B.Paste") (roundrect_rratio 0.212766) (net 3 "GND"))
  (pad "2" smd roundrect (at 1.0375 0 270) (size 1.175 1.45) (layers "B.Cu" "B.Mask" "B.Paste") (roundrect_rratio 0.212766) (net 4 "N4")))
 (gr_rect (start 41 41) (end 93 75) (stroke (width 0.05) (type default)) (fill no) (locked yes) (layer "Edge.Cuts"))
 (segment (start 51.31375 54.99375) (end 51.01375 55.29375) (width 0.25) (layer "F.Cu") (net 3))
 (segment (start 89.48 45) (end 91.48 43) (width 0.25) (layer "F.Cu") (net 3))
 (segment (start 44.01375 57.44625) (end 43.22 58.24) (width 0.25) (layer "F.Cu") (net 3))
 (segment (start 63.5 55.5) (end 62.60525 56.39475) (width 0.25) (layer "F.Cu") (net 3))
 (segment (start 66.02 49.5) (end 66.02 51.3) (width 0.25) (layer "F.Cu") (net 3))
 (segment (start 66.02 51.3) (end 64.32 53) (width 0.25) (layer "F.Cu") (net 3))
 (segment (start 85.395 51.575) (end 84.5 50.68) (width 0.25) (layer "F.Cu") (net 3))
 (segment (start 84.5 50.68) (end 84.5 48) (width 0.25) (layer "F.Cu") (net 3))
 (segment (start 44.01375 54.29375) (end 44.01375 57.44625) (width 0.25) (layer "F.Cu") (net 3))
 (segment (start 66.32 55) (end 68.82 55) (width 0.25) (layer "F.Cu") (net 3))
 (segment (start 56.71375 54.99375) (end 51.31375 54.99375) (width 0.25) (layer "F.Cu") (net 3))
 (segment (start 45.01375 55.29375) (end 44.01375 54.29375) (width 0.25) (layer "F.Cu") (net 3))
 (segment (start 64 53) (end 63.5 53.5) (width 0.25) (layer "F.Cu") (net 3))
 (segment (start 56.71375 54.99375) (end 58.11475 56.39475) (width 0.25) (layer "F.Cu") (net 3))
 (segment (start 87.5 45) (end 89.48 45) (width 0.25) (layer "F.Cu") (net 3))
 (segment (start 64.32 53) (end 64 53) (width 0.25) (layer "F.Cu") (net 3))
 (segment (start 62.60525 56.39475) (end 58.11475 56.39475) (width 0.25) (layer "F.Cu") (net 3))
 (segment (start 84.5 48) (end 87.5 45) (width 0.25) (layer "F.Cu") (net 3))
 (segment (start 51.01375 55.29375) (end 45.01375 55.29375) (width 0.25) (layer "F.Cu") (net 3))
 (segment (start 86.32 51.575) (end 85.395 51.575) (width 0.25) (layer "F.Cu") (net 3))
 (segment (start 63.5 53.5) (end 63.5 55.5) (width 0.25) (layer "F.Cu") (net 3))
 (segment (start 64.32 53) (end 66.32 55) (width 0.25) (layer "F.Cu") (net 3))
 (via (at 86.5 51.5) (size 0.6) (drill 0.3) (layers "F.Cu" "B.Cu") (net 3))
 (segment (start 87.5 73) (end 87.5 71) (width 0.25) (layer "B.Cu") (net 3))
 (segment (start 64 73) (end 65 74) (width 0.25) (layer "B.Cu") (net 3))
 (segment (start 72.336 57.38463) (end 72.336 63.664) (width 0.25) (layer "B.Cu") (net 3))
 (segment (start 69.95137 55) (end 72.336 57.38463) (width 0.25) (layer "B.Cu") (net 3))
 (segment (start 87.764 61.064) (end 87.764 52.764) (width 0.25) (layer "B.Cu") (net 3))
 (segment (start 86.5 74) (end 87.5 73) (width 0.25) (layer "B.Cu") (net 3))
 (segment (start 72.336 63.664) (end 71.5 64.5) (width 0.25) (layer "B.Cu") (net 3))
 (segment (start 53.3 63) (end 52.204 61.904) (width 0.25) (layer "B.Cu") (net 3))
 (segment (start 52.204 61.904) (end 52.204 56.484) (width 0.25) (layer "B.Cu") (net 3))
 (segment (start 89.7 68.8) (end 89.7 63) (width 0.25) (layer "B.Cu") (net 3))
 (segment (start 68.82 55) (end 69.95137 55) (width 0.25) (layer "B.Cu") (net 3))
 (segment (start 71.5 64.5) (end 70.5 64.5) (width 0.25) (layer "B.Cu") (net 3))
 (segment (start 52.204 56.484) (end 51.01375 55.29375) (width 0.25) (layer "B.Cu") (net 3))
 (segment (start 87.5 71) (end 89.7 68.8) (width 0.25) (layer "B.Cu") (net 3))
 (segment (start 87.764 52.764) (end 86.5 51.5) (width 0.25) (layer "B.Cu") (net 3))
 (segment (start 65 74) (end 86.5 74) (width 0.25) (layer "B.Cu") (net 3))
 (segment (start 89.7 63) (end 87.764 61.064) (width 0.25) (layer "B.Cu") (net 3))
 (segment (start 43.5 61.5) (end 43.5 58.52) (width 0.25) (layer "B.Cu") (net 3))
 (segment (start 53.3 63) (end 53.3 64.9) (width 0.25) (layer "B.Cu") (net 3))
 (segment (start 70.5 64.5) (end 64 71) (width 0.25) (layer "B.Cu") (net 3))
 (segment (start 64 71) (end 64 73) (width 0.25) (layer "B.Cu") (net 3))
 (segment (start 53.3 64.9) (end 48.7 69.5) (width 0.25) (layer "B.Cu") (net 3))
 (segment (start 43.5 58.52) (end 43.22 58.24) (width 0.25) (layer "B.Cu") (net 3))
 (segment (start 63.9 66.5) (end 64 66.5) (width 0.25) (layer "B.Cu") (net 2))
 (segment (start 63.9 66.5) (end 59.4 71) (width 0.25) (layer "B.Cu") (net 2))
 (segment (start 64.5 66) (end 64.5 62.36) (width 0.25) (layer "B.Cu") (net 2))
 (segment (start 68.62 58.24) (end 64.5 62.36) (width 0.25) (layer "B.Cu") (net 2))
 (segment (start 64 66.5) (end 64.5 66) (width 0.25) (layer "B.Cu") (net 2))
 (segment (start 80.5 68.8) (end 78.3 71) (width 1) (layer "F.Cu") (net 1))
 (segment (start 78.3 71) (end 68.8 71) (width 1) (layer "F.Cu") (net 1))
 (segment (start 68.8 71) (end 62.3 64.5) (width 1) (layer "F.Cu") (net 1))
 (segment (start 80.5 63) (end 80.5 68.8) (width 1) (layer "F.Cu") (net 1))
 (segment (start 91.48 58.24) (end 89.72 60) (width 1) (layer "F.Cu") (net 1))
 (segment (start 91.4 51.904) (end 91.346 51.85) (width 1) (layer "F.Cu") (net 1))
 (segment (start 91.4 55) (end 91.4 51.904) (width 1) (layer "F.Cu") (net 1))
 (segment (start 91.48 55.08) (end 91.4 55) (width 1) (layer "F.Cu") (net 1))
 (segment (start 60 64.5) (end 54.8 69.7) (width 1) (layer "F.Cu") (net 1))
 (segment (start 91.48 58.24) (end 91.48 55.08) (width 1) (layer "F.Cu") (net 1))
 (segment (start 83.5 60) (end 80.5 63) (width 1) (layer "F.Cu") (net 1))
 (segment (start 62.3 64.5) (end 60 64.5) (width 1) (layer "F.Cu") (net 1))
 (segment (start 55.8 71) (end 54.8 71) (width 1) (layer "F.Cu") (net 1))
 (segment (start 54.8 69.7) (end 54.8 71) (width 1) (layer "F.Cu") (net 1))
 (segment (start 89.72 60) (end 83.5 60) (width 1) (layer "F.Cu") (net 1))
 (segment (start 46.93375 44.17375) (end 45.76 43) (width 0.25) (layer "F.Cu") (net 18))
 (segment (start 46.93375 46.99375) (end 46.93375 44.17375) (width 0.25) (layer "F.Cu") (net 18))
 (segment (start 43.22 43) (end 43.22 48.9) (width 0.25) (layer "F.Cu") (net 17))
 (segment (start 43.22 48.9) (end 44.01375 49.69375) (width 0.25) (layer "F.Cu") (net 17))
 (segment (start 77.9 46) (end 79.273 44.627) (width 0.25) (layer "F.Cu") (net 33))
 (segment (start 79.273 44.627) (end 84.773 44.627) (width 0.25) (layer "F.Cu") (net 33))
 (segment (start 84.773 44.627) (end 86.4 43) (width 0.25) (layer "F.Cu") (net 33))
 (segment (start 73.7 61.8) (end 82.9 71) (width 0.25) (layer "B.Cu") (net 13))
 (segment (start 73.7 58.24) (end 73.7 61.8) (width 0.25) (layer "B.Cu") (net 13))
 (segment (start 76.7825 49) (end 76.774 48.9915) (width 0.25) (layer "F.Cu") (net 9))
 (segment (start 76.7825 48.7825) (end 76 48) (width 0.25) (layer "F.Cu") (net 9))
 (segment (start 76 48) (end 76 45.82) (width 0.25) (layer "F.Cu") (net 9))
 (segment (start 80.144 44.176) (end 81.32 43) (width 0.25) (layer "F.Cu") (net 9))
 (segment (start 76.7825 49) (end 76.7825 48.7825) (width 0.25) (layer "F.Cu") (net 9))
 (segment (start 77.644 44.176) (end 80.144 44.176) (width 0.25) (layer "F.Cu") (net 9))
 (segment (start 76 45.82) (end 77.644 44.176) (width 0.25) (layer "F.Cu") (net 9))
 (segment (start 66.9 62.5) (end 66.9 64.5) (width 0.25) (layer "B.Cu") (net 10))
 (segment (start 71.16 58.24) (end 66.9 62.5) (width 0.25) (layer "B.Cu") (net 10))
 (segment (start 76.24 58.24) (end 76.24 60.24) (width 0.25) (layer "B.Cu") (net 16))
 (segment (start 77 61) (end 83.1 61) (width 0.25) (layer "B.Cu") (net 16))
 (segment (start 83.1 61) (end 85.1 63) (width 0.25) (layer "B.Cu") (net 16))
 (segment (start 76.24 60.24) (end 77 61) (width 0.25) (layer "B.Cu") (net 16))
 (segment (start 79.7075 50.575) (end 81.2825 49) (width 0.25) (layer "F.Cu") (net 11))
 (segment (start 71.695 50.575) (end 79.7075 50.575) (width 0.25) (layer "F.Cu") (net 11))
 (segment (start 70.62 49.5) (end 71.695 50.575) (width 0.25) (layer "F.Cu") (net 11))
 (segment (start 84.779999 52.799999) (end 88.420001 52.799999) (width 0.25) (layer "F.Cu") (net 5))
 (segment (start 83.98 52) (end 83.98 49.6225) (width 0.25) (layer "F.Cu") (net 5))
 (segment (start 83.98 49.6225) (end 83.3575 49) (width 0.25) (layer "F.Cu") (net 5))
 (segment (start 88.420001 52.799999) (end 89.37 51.85) (width 0.25) (layer "F.Cu") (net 5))
 (segment (start 83.98 52) (end 84.779999 52.799999) (width 0.25) (layer "F.Cu") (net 5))
 (segment (start 78.8575 48.3825) (end 78.8575 49) (width 0.25) (layer "F.Cu") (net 8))
 (segment (start 81.24 46) (end 78.8575 48.3825) (width 0.25) (layer "F.Cu") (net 8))
 (segment (start 73.82 52) (end 73.32 52) (width 0.25) (layer "F.Cu") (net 12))
 (segment (start 78.98 55) (end 78.82 55) (width 0.25) (layer "F.Cu") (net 12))
 (segment (start 73.32 52) (end 72.32 53) (width 0.25) (layer "F.Cu") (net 12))
 (segment (start 72.32 53) (end 66.395 53) (width 0.25) (layer "F.Cu") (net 12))
 (segment (start 81.24 55) (end 78.98 55) (width 0.25) (layer "F.Cu") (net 12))
 (segment (start 75.82 52) (end 73.82 52) (width 0.25) (layer "F.Cu") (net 12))
 (segment (start 78.82 55) (end 75.82 52) (width 0.25) (layer "F.Cu") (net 12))
 (segment (start 61.31375 54.99375) (end 61.32 55) (width 0.25) (layer "F.Cu") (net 14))
 (segment (start 60.82 47.99375) (end 60.82 54.5) (width 0.25) (layer "F.Cu") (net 14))
 (segment (start 60.82 54.5) (end 61.31375 54.99375) (width 0.25) (layer "F.Cu") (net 14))
 (segment (start 67.74 46) (end 60.90125 46) (width 0.25) (layer "F.Cu") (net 15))
 (segment (start 60.90125 46) (end 60.82 45.91875) (width 0.25) (layer "F.Cu") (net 15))
 (segment (start 90.5 47.5) (end 91.27 48.27) (width 0.25) (layer "F.Cu") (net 7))
 (segment (start 86.32 49.18) (end 88 47.5) (width 0.25) (layer "F.Cu") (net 7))
 (segment (start 86.32 49.5) (end 86.32 49.18) (width 0.25) (layer "F.Cu") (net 7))
 (segment (start 88 47.5) (end 90.5 47.5) (width 0.25) (layer "F.Cu") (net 7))
 (segment (start 91.27 48.27) (end 91.27 49.15) (width 0.25) (layer "F.Cu") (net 7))
 (segment (start 54.71375 46.99375) (end 57.09375 46.99375) (width 0.25) (layer "F.Cu") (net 48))
 (segment (start 51.01375 50.69375) (end 54.71375 46.99375) (width 0.25) (layer "F.Cu") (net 48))
 (segment (start 88.1065 50.4135) (end 85.0865 50.4135) (width 0.25) (layer "F.Cu") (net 6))
 (segment (start 85.0865 50.4135) (end 85 50.327) (width 0.25) (layer "F.Cu") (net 6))
 (segment (start 89.37 49.15) (end 88.1065 50.4135) (width 0.25) (layer "F.Cu") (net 6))
 (segment (start 87.13781 46) (end 91.4 46) (width 0.25) (layer "F.Cu") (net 6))
 (segment (start 85 48.13781) (end 87.13781 46) (width 0.25) (layer "F.Cu") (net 6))
 (segment (start 90.32 50.1) (end 90.32 51.85) (width 0.25) (layer "F.Cu") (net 6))
 (segment (start 85 50.327) (end 85 48.13781) (width 0.25) (layer "F.Cu") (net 6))
 (segment (start 89.37 49.15) (end 90.32 50.1) (width 0.25) (layer "F.Cu") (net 6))
 (segment (start 43.3 69.5) (end 43.3 63.775) (width 0.25) (layer "B.Cu") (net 4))
 (segment (start 43.5 69.3) (end 43.3 69.5) (width 0.25) (layer "B.Cu") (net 4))
 (segment (start 48.125 63.575) (end 48.7 63) (width 0.25) (layer "B.Cu") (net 4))
 (segment (start 43.3 63.775) (end 43.5 63.575) (width 0.25) (layer "B.Cu") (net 4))
 (segment (start 43.5 63.575) (end 48.125 63.575) (width 0.25) (layer "B.Cu") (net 4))
 (segment (start 48.7 63) (end 48.7 61.18) (width 0.25) (layer "B.Cu") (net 4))
 (segment (start 48.7 61.18) (end 45.76 58.24) (width 0.25) (layer "B.Cu") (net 4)))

